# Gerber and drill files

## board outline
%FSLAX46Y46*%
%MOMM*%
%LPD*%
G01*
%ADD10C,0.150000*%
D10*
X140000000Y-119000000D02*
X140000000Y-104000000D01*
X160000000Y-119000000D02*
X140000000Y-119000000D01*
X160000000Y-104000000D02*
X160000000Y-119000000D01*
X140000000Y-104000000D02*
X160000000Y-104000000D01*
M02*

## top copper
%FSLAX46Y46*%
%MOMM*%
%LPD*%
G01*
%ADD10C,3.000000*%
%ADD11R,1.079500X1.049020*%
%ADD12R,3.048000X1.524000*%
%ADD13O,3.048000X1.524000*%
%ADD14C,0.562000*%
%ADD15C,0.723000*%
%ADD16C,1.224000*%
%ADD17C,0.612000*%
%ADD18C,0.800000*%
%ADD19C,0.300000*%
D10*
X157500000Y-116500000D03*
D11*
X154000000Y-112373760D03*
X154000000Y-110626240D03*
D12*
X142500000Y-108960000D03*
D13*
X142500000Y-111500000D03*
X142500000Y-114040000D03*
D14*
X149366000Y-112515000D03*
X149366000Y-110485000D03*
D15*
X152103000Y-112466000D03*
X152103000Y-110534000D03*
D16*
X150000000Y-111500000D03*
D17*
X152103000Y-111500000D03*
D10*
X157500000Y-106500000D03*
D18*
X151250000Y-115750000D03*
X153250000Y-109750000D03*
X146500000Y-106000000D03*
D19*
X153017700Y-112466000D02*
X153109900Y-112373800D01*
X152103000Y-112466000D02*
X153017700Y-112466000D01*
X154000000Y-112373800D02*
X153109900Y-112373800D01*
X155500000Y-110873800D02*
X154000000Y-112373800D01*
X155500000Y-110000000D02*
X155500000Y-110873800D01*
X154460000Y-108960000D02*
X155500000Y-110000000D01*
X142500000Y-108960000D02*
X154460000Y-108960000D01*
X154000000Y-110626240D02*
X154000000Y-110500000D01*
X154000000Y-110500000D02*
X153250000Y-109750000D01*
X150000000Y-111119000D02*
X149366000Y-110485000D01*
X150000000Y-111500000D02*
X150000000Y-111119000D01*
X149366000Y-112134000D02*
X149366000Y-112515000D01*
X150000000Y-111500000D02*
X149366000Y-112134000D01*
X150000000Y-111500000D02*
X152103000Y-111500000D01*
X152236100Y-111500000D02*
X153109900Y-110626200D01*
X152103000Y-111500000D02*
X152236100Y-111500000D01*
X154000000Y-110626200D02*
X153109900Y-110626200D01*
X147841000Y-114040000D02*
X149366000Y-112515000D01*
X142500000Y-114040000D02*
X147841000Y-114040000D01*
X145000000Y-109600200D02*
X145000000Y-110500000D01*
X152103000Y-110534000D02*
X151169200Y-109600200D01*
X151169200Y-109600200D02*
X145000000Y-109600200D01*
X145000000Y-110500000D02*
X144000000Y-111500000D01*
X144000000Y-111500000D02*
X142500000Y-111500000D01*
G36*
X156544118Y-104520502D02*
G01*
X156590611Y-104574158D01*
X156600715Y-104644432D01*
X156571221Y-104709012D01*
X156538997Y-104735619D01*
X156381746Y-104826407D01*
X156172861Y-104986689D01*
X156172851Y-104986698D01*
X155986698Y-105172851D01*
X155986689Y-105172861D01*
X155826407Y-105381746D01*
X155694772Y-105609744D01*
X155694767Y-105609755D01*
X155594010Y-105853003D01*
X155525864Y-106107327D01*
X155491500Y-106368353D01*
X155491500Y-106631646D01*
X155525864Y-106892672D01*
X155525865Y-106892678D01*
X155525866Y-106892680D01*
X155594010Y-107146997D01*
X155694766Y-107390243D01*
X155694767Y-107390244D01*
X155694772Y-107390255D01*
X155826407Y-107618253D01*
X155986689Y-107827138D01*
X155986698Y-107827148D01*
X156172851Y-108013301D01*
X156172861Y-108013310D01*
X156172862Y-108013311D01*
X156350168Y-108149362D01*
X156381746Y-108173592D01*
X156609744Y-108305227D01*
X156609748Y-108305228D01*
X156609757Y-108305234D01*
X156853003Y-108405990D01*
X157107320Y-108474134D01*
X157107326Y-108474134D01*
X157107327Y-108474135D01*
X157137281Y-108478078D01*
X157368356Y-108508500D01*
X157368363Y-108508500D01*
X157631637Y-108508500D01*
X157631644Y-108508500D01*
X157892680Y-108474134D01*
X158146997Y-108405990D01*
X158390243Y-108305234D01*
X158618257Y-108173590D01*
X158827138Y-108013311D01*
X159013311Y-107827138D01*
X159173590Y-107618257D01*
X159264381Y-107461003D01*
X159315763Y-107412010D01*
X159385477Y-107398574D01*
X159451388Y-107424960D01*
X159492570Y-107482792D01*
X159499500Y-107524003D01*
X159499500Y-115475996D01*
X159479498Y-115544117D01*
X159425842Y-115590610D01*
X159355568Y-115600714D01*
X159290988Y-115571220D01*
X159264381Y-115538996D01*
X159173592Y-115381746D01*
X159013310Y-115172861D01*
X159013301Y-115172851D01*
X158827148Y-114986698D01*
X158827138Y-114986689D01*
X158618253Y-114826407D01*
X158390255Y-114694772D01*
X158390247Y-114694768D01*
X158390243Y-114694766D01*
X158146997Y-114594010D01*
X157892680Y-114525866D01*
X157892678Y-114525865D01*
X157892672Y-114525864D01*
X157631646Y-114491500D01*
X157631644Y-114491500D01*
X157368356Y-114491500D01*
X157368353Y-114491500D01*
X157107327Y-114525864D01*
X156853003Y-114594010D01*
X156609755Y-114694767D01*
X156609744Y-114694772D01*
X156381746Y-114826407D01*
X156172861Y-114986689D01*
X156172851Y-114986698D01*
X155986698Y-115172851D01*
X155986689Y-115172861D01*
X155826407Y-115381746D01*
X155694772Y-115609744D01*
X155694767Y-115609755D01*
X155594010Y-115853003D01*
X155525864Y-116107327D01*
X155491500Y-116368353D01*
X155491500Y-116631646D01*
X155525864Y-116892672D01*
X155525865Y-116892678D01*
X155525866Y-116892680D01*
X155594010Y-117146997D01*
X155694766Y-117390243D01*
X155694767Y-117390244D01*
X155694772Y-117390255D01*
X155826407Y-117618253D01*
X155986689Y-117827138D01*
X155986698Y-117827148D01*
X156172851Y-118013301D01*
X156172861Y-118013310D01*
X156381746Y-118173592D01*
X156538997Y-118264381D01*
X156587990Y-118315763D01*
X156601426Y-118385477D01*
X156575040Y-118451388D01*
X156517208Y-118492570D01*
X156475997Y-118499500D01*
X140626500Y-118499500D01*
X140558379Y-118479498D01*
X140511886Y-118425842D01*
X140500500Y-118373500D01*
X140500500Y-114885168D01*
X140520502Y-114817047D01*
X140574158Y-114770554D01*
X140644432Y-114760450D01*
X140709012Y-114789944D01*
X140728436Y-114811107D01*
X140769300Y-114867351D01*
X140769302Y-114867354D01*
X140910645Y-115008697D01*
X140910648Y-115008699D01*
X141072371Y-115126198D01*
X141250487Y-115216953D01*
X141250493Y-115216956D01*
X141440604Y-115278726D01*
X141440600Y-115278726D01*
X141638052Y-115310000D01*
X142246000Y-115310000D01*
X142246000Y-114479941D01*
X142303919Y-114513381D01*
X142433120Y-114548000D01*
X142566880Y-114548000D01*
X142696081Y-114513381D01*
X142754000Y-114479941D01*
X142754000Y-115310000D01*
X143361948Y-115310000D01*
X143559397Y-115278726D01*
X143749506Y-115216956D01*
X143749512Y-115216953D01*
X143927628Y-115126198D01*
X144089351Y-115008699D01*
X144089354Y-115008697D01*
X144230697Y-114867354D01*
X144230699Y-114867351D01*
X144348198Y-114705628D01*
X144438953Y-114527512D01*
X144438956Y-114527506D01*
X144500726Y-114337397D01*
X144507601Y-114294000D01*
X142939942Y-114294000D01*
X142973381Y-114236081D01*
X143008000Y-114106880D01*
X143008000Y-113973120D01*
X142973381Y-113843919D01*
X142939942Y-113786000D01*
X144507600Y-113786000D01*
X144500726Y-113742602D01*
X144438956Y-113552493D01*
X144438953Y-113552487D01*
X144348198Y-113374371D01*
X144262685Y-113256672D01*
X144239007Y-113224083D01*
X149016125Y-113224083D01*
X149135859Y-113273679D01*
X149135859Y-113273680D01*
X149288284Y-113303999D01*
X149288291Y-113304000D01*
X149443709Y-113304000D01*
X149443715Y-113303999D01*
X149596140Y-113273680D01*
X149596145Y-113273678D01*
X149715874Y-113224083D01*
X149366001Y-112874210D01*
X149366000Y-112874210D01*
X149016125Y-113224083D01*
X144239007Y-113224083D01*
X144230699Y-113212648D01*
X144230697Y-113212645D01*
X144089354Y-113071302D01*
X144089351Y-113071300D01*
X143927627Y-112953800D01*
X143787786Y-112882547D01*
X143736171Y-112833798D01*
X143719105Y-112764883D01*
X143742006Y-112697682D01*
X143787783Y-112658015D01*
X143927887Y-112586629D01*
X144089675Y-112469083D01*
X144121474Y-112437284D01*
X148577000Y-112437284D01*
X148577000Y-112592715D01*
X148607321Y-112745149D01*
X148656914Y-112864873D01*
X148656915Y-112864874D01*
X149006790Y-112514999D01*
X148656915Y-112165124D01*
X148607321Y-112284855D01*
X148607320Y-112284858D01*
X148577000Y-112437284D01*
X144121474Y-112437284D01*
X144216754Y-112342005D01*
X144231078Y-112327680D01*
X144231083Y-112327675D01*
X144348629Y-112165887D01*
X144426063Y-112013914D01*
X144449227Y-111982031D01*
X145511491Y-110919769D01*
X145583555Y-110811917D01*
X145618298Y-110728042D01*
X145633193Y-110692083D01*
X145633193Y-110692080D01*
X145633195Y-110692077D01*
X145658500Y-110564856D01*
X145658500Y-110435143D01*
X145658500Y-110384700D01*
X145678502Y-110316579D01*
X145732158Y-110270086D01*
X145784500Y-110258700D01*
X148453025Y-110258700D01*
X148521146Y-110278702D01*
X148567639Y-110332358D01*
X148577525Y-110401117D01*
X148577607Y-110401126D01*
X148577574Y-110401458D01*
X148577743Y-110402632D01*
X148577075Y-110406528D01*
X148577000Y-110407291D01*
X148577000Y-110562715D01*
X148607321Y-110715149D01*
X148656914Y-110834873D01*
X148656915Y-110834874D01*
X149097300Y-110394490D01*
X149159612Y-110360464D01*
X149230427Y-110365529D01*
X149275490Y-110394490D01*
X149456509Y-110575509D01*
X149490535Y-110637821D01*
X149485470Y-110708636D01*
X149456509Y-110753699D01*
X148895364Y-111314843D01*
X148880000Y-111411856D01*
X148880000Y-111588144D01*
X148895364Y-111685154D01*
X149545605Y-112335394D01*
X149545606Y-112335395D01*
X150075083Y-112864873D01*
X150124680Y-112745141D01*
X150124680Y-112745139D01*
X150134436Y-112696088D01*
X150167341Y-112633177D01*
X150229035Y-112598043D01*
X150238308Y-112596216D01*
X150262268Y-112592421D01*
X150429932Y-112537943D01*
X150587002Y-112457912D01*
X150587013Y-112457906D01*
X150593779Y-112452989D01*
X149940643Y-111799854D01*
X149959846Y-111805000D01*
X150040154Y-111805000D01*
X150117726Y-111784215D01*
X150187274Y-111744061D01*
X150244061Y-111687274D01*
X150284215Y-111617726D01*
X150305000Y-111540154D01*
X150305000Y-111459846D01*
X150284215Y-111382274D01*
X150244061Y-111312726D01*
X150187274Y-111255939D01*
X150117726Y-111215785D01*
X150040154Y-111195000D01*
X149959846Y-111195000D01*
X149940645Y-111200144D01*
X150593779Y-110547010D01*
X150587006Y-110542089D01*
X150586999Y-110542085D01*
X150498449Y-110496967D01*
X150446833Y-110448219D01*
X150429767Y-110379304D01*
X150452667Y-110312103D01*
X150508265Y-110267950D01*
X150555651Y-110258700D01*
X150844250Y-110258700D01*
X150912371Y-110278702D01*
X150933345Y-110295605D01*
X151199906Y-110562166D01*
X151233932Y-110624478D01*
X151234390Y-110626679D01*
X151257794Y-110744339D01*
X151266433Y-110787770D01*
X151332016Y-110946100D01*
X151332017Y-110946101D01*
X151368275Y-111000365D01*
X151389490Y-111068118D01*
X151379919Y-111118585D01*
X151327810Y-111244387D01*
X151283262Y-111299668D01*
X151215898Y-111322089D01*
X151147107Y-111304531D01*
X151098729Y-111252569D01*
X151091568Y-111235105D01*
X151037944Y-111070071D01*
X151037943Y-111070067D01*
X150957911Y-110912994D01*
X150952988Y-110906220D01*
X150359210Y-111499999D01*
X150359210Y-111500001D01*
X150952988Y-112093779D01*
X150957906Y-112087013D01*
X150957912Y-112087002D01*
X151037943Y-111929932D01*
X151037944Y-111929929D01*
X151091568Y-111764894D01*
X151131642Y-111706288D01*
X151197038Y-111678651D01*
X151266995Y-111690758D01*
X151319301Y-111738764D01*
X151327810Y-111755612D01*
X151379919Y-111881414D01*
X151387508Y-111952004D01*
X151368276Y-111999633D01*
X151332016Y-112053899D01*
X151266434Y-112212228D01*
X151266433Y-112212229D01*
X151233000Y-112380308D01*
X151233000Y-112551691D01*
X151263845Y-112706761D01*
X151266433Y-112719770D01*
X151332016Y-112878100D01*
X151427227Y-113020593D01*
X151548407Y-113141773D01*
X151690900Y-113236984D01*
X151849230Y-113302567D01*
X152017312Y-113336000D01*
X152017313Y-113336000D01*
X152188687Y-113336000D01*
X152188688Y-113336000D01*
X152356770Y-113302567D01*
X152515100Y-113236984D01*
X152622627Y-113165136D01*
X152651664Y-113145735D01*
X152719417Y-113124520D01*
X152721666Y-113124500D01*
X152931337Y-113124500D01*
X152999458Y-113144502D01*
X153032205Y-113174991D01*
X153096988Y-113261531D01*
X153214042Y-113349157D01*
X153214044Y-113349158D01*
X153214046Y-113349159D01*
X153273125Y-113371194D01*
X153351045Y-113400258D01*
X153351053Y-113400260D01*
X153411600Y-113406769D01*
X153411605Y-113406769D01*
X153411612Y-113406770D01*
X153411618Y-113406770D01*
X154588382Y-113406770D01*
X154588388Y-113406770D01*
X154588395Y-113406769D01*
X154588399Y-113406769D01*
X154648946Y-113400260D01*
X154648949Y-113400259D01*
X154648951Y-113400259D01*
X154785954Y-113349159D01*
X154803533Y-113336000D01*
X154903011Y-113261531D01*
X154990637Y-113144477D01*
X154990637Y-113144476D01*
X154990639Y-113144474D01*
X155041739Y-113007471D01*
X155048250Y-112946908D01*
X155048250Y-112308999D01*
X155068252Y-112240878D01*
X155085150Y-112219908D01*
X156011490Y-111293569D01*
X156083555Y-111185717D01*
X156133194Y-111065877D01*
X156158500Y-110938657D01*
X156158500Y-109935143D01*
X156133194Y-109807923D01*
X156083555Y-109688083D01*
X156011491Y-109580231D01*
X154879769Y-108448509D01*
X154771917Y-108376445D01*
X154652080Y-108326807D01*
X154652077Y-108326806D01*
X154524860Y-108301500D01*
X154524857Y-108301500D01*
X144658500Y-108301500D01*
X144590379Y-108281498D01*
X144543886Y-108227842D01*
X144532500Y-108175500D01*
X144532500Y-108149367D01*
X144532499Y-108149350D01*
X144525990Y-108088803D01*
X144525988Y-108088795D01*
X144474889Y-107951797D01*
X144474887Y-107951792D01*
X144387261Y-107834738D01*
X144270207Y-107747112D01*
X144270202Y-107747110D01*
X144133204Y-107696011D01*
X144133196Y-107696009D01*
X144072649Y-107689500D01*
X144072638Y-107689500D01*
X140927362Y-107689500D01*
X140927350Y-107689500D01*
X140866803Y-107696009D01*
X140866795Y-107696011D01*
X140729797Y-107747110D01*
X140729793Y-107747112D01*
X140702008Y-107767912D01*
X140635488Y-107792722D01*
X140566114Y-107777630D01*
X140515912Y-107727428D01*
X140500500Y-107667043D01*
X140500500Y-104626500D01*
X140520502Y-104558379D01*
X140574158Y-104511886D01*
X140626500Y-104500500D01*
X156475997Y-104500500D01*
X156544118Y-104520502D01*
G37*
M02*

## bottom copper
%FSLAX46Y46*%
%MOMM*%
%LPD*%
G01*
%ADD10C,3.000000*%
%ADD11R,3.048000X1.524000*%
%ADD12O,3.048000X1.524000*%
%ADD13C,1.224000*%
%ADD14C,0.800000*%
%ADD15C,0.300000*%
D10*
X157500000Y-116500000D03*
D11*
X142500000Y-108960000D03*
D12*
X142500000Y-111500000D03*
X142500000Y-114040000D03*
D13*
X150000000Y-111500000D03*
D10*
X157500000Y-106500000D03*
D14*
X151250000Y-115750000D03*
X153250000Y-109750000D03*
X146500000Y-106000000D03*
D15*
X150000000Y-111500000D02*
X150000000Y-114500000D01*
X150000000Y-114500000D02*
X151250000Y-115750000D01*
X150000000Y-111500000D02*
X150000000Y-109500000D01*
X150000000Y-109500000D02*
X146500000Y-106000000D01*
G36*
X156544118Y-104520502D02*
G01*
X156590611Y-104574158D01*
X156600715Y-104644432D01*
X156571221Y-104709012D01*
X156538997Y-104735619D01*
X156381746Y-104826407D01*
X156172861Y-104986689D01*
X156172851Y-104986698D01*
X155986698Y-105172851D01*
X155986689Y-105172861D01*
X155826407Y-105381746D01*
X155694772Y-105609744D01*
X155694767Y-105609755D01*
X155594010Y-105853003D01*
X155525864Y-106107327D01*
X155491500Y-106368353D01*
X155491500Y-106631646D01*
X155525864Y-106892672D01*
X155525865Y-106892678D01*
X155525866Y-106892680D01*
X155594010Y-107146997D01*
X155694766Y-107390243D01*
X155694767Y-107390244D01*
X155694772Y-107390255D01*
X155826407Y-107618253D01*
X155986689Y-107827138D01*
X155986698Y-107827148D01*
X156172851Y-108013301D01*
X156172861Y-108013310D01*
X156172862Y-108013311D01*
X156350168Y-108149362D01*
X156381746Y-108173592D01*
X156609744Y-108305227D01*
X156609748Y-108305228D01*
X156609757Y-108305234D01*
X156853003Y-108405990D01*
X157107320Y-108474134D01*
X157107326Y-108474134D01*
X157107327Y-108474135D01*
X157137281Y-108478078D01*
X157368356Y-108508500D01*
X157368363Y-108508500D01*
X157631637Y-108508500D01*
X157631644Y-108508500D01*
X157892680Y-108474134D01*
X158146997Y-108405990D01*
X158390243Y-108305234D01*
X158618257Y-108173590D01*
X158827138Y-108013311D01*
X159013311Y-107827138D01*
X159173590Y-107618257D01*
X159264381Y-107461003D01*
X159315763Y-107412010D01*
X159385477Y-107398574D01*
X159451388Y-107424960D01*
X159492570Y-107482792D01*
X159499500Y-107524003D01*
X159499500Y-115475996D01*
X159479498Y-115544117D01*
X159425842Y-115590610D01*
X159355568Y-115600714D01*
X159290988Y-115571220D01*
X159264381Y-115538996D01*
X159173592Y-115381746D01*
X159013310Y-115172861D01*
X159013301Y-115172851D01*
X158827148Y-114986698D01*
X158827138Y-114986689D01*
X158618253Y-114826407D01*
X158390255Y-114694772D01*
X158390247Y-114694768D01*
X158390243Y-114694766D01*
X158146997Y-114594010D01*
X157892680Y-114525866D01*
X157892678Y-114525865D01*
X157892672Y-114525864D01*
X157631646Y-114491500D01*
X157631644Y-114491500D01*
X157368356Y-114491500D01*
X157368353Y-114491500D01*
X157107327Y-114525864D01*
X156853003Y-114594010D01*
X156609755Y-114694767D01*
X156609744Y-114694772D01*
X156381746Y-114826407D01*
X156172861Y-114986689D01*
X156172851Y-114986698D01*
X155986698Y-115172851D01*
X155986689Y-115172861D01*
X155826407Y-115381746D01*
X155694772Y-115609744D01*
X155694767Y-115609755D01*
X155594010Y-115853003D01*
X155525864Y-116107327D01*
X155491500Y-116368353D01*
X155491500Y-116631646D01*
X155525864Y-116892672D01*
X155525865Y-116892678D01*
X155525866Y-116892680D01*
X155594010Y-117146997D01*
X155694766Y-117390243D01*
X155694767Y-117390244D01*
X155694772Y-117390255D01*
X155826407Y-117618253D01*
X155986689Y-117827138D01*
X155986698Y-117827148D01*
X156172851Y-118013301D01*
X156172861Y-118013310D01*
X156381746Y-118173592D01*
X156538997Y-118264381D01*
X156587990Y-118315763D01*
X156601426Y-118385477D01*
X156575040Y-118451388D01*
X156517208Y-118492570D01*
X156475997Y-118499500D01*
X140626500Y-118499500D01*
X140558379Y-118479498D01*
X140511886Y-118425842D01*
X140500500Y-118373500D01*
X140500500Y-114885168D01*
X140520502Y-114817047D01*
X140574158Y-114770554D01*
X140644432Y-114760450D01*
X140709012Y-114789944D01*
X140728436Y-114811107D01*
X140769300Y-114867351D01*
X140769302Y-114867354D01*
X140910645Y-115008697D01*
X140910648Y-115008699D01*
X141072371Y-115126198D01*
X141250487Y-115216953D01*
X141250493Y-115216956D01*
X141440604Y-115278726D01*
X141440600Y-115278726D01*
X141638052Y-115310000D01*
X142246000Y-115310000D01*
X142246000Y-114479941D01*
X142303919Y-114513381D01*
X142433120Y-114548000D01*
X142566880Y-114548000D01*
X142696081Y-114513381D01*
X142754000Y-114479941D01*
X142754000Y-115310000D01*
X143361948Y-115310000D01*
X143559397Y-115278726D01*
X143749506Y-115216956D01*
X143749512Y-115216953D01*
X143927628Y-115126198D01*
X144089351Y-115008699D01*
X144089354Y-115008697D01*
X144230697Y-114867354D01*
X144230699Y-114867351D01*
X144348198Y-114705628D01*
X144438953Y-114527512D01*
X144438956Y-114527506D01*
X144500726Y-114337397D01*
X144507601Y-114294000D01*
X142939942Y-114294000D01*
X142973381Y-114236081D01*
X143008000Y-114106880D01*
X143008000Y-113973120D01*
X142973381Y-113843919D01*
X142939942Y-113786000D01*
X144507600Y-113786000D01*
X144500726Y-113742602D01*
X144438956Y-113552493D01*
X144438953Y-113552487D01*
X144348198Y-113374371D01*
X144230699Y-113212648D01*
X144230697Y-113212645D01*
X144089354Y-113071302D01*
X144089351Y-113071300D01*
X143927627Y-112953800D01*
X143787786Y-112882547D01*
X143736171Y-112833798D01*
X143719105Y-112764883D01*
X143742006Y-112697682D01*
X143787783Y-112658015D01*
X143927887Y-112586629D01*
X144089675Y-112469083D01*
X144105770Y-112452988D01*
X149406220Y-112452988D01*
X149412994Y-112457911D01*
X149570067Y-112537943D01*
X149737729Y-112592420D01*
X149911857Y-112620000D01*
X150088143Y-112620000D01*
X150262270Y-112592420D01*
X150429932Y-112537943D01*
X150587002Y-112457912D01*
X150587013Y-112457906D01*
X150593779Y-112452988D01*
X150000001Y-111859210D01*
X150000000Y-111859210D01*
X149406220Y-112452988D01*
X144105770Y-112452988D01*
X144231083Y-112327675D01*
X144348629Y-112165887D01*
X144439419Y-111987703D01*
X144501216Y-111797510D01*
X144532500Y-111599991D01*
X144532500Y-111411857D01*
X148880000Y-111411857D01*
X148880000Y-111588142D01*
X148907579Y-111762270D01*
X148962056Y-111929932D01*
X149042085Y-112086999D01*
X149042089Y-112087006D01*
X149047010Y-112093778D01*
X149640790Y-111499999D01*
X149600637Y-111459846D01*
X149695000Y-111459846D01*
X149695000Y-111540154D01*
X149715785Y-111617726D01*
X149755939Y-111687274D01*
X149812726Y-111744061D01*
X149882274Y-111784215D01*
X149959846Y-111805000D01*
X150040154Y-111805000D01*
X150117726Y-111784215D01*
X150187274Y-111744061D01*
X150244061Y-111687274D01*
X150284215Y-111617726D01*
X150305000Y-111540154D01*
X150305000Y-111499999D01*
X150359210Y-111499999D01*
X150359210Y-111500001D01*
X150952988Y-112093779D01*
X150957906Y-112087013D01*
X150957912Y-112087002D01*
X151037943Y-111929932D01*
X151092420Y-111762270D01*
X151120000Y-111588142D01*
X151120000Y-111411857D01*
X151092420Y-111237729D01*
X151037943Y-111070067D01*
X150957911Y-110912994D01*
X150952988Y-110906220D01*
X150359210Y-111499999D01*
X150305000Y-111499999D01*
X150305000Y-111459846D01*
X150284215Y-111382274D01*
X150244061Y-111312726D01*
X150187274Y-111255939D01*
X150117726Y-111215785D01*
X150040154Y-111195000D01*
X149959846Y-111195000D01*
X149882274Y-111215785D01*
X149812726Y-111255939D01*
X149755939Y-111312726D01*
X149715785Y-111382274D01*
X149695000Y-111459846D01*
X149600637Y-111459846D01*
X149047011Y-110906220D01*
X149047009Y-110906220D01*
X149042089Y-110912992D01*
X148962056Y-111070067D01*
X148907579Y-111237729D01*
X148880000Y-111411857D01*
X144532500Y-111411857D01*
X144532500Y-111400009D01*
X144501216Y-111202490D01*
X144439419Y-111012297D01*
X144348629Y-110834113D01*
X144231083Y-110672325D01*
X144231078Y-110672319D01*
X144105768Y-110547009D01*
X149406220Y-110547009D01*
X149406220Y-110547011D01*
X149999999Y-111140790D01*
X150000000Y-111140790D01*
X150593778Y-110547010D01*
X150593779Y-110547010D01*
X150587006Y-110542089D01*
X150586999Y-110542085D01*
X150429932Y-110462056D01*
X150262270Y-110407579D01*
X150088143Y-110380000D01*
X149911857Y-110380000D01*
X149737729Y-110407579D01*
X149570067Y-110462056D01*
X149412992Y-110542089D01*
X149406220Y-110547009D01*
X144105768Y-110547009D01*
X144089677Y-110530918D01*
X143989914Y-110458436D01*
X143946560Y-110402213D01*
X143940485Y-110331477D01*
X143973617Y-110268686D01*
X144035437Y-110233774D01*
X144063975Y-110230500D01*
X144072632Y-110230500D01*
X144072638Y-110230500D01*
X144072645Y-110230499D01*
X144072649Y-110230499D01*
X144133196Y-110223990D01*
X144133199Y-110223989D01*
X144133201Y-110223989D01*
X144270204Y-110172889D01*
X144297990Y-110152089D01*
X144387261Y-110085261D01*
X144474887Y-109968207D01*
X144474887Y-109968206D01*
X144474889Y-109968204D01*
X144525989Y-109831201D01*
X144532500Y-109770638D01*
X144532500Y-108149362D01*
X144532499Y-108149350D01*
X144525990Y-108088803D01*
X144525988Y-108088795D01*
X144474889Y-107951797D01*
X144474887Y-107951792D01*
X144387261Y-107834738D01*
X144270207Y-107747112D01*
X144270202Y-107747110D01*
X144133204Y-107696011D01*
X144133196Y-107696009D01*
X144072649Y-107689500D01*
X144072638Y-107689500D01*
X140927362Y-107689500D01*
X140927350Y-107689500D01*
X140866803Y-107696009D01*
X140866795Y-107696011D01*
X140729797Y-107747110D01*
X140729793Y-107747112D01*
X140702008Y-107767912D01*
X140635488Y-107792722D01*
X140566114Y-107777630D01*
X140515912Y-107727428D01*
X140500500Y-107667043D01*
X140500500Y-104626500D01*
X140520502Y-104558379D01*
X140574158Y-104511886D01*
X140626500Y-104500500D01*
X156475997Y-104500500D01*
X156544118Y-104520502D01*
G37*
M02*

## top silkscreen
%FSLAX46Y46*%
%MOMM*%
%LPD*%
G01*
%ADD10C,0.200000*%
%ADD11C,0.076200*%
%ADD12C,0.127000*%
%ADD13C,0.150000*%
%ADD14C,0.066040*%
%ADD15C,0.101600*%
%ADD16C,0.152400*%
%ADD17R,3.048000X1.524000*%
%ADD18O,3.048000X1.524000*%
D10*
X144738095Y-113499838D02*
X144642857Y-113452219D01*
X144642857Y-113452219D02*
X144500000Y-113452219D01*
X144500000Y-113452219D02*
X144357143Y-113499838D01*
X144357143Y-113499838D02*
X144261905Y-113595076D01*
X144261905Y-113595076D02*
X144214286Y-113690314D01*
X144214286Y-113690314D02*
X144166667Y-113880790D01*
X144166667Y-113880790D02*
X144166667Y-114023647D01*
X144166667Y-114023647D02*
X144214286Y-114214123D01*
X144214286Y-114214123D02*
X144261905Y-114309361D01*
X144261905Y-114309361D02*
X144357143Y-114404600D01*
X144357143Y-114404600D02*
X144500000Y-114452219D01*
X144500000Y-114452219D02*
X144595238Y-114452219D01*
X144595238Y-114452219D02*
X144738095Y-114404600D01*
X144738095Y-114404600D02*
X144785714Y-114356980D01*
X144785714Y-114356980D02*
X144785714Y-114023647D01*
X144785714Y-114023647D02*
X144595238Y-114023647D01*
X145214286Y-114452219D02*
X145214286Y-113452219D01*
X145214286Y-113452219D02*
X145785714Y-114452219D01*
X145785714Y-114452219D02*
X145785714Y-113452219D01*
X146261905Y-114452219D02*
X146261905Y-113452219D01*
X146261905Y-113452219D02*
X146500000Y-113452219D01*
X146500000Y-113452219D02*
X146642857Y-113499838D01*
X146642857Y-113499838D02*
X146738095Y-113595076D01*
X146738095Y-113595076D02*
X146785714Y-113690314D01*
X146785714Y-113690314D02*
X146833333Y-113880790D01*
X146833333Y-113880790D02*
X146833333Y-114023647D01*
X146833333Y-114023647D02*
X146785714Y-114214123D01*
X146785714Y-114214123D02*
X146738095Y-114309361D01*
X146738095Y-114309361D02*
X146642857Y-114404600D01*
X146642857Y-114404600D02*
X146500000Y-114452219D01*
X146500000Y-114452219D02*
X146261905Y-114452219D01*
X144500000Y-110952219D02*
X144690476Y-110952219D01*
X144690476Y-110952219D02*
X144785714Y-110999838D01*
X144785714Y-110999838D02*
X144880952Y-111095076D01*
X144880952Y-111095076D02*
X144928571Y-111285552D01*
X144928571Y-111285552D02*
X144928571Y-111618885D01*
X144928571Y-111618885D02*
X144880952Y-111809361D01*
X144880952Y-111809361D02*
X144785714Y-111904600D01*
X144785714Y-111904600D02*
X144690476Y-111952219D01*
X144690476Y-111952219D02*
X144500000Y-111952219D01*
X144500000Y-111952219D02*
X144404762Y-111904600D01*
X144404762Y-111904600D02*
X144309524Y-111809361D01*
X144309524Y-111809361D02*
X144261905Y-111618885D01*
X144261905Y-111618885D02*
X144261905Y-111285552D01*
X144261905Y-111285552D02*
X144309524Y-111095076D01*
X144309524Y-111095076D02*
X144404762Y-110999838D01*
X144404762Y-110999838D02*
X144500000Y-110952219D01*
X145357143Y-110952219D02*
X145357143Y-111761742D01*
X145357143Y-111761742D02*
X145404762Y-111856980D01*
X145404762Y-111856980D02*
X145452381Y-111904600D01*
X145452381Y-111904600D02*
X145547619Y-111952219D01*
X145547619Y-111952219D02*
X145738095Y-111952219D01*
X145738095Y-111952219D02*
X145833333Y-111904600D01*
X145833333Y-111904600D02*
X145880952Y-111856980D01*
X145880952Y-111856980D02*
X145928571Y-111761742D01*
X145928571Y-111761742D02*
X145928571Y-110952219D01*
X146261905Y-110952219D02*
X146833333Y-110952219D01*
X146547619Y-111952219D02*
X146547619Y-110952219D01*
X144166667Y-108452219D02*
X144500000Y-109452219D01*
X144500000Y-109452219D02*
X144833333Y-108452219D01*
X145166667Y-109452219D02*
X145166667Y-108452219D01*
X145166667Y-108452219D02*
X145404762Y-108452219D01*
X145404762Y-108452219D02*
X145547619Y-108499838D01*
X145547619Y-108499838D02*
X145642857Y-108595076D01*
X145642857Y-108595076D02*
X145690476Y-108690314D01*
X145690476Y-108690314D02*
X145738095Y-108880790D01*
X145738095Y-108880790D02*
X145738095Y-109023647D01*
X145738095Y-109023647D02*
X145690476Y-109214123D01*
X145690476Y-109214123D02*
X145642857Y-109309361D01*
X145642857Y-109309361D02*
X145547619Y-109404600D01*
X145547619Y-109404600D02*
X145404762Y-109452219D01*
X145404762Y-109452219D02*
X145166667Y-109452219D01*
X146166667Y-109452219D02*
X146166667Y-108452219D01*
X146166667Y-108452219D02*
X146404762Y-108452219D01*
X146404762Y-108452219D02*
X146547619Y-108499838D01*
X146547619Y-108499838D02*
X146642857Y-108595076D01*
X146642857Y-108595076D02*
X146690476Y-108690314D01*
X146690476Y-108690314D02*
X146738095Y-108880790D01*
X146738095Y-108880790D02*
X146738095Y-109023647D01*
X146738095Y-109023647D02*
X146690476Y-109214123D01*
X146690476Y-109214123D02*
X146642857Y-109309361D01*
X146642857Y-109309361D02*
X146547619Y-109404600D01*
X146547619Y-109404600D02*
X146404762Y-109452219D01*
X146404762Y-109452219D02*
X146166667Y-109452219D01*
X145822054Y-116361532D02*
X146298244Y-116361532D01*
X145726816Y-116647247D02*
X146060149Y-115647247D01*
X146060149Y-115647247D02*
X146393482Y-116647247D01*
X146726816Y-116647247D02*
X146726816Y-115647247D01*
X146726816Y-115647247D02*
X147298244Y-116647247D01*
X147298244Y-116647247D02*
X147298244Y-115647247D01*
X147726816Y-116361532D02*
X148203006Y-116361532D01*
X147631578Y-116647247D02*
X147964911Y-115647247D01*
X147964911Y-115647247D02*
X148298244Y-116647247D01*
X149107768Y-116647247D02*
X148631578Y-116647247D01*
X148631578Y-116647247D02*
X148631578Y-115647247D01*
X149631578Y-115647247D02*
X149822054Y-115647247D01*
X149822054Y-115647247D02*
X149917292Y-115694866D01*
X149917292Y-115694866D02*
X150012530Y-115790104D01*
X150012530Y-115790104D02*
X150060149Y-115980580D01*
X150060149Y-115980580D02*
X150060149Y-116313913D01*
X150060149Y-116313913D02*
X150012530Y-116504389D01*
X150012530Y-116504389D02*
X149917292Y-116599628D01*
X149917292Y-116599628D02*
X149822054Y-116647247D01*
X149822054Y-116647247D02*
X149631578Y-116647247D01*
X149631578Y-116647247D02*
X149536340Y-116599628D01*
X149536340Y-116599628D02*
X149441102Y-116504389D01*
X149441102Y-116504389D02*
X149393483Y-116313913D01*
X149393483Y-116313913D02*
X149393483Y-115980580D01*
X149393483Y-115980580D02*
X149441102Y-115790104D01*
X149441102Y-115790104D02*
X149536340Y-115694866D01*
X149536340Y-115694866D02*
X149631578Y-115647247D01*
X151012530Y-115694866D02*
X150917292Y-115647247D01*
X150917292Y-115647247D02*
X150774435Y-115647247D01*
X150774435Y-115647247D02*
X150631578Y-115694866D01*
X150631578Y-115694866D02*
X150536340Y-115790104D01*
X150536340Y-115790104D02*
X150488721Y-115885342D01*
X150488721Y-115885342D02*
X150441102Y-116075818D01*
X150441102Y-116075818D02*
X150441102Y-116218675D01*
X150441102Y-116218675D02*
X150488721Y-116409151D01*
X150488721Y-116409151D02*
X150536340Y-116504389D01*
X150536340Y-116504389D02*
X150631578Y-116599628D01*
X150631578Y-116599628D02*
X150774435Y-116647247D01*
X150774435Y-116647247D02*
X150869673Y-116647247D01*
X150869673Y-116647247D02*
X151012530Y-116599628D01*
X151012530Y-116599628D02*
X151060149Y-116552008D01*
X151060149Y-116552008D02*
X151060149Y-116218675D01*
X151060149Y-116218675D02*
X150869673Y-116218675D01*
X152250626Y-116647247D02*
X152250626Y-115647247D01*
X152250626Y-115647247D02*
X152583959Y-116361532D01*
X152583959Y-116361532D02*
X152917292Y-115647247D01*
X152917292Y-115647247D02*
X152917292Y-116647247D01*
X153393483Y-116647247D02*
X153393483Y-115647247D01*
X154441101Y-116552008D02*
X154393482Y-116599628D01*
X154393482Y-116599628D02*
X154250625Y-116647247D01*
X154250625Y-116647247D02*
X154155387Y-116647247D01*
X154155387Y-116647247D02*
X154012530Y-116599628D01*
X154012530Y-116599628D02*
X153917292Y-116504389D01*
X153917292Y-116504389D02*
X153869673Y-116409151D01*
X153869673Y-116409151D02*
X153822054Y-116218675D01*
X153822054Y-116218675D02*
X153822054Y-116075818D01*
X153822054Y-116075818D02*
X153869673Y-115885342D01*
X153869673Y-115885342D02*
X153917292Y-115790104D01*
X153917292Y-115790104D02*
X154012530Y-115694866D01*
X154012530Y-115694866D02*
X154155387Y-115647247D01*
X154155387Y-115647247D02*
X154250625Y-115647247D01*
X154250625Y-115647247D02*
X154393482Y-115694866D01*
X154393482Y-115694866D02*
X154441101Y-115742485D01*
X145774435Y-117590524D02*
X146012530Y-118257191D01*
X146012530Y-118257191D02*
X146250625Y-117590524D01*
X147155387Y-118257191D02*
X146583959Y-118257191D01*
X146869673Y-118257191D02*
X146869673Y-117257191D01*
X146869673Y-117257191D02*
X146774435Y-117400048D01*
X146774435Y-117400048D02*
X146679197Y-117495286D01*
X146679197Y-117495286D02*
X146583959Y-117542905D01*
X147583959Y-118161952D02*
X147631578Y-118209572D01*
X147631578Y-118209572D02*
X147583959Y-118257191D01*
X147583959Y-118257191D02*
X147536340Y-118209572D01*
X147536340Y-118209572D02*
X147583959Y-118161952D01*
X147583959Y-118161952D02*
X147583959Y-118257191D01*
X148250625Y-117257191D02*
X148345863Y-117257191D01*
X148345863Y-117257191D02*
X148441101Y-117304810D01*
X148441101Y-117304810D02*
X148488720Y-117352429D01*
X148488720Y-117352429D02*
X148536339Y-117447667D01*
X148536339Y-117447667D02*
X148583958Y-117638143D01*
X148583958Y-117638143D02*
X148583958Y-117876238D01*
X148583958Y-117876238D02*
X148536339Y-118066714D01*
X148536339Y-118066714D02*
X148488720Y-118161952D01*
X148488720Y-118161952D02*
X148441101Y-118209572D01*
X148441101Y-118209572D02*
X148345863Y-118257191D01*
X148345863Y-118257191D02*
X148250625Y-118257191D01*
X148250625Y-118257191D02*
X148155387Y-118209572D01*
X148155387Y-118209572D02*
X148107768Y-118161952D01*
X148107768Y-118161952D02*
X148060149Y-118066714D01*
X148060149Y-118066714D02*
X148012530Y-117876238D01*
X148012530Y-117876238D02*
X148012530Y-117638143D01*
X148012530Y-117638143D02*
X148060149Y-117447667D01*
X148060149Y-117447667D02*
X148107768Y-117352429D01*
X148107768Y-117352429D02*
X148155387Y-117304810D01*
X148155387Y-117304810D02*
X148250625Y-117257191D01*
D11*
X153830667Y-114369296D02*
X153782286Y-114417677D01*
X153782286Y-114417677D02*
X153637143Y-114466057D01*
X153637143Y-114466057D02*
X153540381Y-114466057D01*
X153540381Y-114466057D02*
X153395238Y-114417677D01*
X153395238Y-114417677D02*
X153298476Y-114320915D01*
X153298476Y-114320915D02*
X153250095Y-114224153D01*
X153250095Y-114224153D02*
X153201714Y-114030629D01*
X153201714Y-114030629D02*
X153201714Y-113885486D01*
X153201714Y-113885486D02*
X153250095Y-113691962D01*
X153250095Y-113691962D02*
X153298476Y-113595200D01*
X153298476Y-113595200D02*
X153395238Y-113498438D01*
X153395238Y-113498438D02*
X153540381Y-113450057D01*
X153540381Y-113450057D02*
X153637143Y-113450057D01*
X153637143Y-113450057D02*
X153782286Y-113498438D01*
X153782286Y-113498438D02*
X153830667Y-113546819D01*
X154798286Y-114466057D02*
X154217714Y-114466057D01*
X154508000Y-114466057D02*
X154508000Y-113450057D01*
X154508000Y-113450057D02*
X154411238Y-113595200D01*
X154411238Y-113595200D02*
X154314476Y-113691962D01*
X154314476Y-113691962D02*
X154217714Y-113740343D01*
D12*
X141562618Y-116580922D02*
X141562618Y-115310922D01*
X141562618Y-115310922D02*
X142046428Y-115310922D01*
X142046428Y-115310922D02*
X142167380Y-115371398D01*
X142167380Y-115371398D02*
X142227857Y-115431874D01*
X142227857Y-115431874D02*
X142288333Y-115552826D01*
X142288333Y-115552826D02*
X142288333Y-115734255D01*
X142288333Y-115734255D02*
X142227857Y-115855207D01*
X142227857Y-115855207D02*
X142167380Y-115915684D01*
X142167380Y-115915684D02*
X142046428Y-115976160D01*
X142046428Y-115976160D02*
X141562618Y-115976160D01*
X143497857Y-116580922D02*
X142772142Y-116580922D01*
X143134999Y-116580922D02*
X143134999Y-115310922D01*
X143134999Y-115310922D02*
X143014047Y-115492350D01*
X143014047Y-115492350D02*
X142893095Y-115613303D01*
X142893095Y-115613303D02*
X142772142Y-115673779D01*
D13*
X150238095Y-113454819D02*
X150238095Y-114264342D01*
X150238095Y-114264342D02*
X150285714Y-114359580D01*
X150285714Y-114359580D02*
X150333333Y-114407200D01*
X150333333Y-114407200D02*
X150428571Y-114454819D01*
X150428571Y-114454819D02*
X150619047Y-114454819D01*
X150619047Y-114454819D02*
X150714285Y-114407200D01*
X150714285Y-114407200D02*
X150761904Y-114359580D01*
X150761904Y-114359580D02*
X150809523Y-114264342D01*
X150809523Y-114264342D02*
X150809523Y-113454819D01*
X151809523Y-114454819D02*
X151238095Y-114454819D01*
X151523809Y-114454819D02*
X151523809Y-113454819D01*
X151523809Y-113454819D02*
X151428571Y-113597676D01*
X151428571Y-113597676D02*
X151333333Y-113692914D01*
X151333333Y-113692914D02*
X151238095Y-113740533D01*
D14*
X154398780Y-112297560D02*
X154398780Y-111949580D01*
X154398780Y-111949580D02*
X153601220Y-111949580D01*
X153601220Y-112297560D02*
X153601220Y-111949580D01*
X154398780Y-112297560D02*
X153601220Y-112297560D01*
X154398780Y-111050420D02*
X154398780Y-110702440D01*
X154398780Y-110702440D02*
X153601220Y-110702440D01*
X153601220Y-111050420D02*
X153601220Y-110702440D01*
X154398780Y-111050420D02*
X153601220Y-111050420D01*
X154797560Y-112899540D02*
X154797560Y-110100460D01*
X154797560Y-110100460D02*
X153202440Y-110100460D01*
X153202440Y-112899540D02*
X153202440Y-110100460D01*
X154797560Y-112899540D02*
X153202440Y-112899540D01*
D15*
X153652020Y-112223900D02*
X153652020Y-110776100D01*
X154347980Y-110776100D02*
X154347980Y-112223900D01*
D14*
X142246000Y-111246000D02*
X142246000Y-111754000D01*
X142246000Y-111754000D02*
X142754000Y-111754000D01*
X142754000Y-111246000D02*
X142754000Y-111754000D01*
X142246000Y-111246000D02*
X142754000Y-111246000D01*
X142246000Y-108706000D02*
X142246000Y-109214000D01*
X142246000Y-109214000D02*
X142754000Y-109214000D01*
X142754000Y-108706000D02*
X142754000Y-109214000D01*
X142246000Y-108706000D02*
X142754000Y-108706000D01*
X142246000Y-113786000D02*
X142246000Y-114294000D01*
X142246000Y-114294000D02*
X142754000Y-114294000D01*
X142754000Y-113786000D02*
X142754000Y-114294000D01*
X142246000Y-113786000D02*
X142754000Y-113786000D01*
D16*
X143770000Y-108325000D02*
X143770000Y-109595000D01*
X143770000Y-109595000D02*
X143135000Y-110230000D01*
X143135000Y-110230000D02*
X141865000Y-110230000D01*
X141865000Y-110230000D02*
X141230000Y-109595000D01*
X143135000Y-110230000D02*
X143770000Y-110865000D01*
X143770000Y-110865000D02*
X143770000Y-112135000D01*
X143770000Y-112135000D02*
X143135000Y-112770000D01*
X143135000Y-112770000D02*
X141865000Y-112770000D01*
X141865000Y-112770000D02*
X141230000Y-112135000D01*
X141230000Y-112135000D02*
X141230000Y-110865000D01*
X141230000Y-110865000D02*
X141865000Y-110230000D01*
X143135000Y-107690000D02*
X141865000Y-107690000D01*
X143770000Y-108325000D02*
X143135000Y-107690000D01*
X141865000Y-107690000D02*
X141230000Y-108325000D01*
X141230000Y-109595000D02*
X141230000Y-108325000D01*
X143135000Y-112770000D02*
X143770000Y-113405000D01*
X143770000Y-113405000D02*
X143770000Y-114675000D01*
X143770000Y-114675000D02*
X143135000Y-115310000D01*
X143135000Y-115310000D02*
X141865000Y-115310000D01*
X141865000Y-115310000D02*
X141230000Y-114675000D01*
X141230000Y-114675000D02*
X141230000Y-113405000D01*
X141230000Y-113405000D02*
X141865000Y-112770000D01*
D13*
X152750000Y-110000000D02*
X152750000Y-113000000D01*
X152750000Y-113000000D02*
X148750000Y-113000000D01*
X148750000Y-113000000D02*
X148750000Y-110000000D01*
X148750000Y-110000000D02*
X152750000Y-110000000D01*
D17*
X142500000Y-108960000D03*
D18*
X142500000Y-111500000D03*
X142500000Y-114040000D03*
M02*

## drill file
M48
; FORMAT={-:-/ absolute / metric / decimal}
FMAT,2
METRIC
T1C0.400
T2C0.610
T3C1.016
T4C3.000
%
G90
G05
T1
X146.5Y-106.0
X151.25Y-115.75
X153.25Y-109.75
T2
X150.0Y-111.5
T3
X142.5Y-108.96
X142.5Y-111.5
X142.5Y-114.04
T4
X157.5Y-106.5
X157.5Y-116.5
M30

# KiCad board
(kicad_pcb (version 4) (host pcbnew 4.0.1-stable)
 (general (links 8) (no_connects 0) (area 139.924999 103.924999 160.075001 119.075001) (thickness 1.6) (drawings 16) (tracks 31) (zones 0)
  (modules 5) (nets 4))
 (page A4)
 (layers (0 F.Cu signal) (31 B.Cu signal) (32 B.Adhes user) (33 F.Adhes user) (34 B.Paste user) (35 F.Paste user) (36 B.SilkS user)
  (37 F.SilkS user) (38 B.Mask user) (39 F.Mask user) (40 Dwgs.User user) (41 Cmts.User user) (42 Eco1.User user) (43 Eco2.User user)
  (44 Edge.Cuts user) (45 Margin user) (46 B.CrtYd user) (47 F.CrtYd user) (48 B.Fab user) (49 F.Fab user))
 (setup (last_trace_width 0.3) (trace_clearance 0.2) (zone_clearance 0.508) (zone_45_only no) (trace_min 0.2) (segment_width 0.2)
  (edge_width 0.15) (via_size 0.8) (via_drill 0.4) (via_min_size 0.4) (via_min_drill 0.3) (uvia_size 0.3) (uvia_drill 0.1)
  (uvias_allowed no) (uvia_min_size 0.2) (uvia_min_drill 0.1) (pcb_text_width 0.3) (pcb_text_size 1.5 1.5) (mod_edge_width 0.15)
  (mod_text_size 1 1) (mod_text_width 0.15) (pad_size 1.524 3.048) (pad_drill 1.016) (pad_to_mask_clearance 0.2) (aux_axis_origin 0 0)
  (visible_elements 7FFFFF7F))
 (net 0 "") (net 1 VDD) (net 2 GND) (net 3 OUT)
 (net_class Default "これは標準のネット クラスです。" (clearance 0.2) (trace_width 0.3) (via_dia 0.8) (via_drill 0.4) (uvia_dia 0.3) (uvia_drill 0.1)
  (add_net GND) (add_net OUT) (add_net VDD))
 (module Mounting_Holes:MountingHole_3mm (layer F.Cu) (at 157.5 116.5)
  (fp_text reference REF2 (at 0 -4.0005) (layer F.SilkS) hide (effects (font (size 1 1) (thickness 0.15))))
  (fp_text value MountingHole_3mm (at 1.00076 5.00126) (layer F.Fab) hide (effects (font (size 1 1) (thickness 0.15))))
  (pad 1 thru_hole circle (at 0 0) (size 3 3) (drill 3) (layers)))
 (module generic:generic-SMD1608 (layer F.Cu) (at 154 111.5 90)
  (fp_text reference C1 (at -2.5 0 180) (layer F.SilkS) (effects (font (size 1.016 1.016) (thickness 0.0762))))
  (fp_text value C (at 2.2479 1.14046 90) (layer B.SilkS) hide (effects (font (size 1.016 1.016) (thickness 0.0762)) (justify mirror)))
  (fp_line (start -0.79756 0.39878) (end -0.44958 0.39878) (layer F.SilkS) (width 0.06604))
  (fp_line (start -0.44958 0.39878) (end -0.44958 -0.39878) (layer F.SilkS) (width 0.06604))
  (fp_line (start -0.79756 -0.39878) (end -0.44958 -0.39878) (layer F.SilkS) (width 0.06604))
  (fp_line (start -0.79756 0.39878) (end -0.79756 -0.39878) (layer F.SilkS) (width 0.06604))
  (fp_line (start 0.44958 0.39878) (end 0.79756 0.39878) (layer F.SilkS) (width 0.06604))
  (fp_line (start 0.79756 0.39878) (end 0.79756 -0.39878) (layer F.SilkS) (width 0.06604))
  (fp_line (start 0.44958 -0.39878) (end 0.79756 -0.39878) (layer F.SilkS) (width 0.06604))
  (fp_line (start 0.44958 0.39878) (end 0.44958 -0.39878) (layer F.SilkS) (width 0.06604))
  (fp_line (start -1.39954 0.79756) (end 1.39954 0.79756) (layer F.SilkS) (width 0.06604))
  (fp_line (start 1.39954 0.79756) (end 1.39954 -0.79756) (layer F.SilkS) (width 0.06604))
  (fp_line (start -1.39954 -0.79756) (end 1.39954 -0.79756) (layer F.SilkS) (width 0.06604))
  (fp_line (start -1.39954 0.79756) (end -1.39954 -0.79756) (layer F.SilkS) (width 0.06604))
  (fp_line (start -0.7239 -0.34798) (end 0.7239 -0.34798) (layer F.SilkS) (width 0.1016))
  (fp_line (start 0.7239 0.34798) (end -0.7239 0.34798) (layer F.SilkS) (width 0.1016))
  (pad 1 smd rect (at -0.87376 0 90) (size 1.04902 1.0795) (layers F.Cu F.Paste F.Mask) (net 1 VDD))
  (pad 2 smd rect (at 0.87376 0 90) (size 1.04902 1.0795) (layers F.Cu F.Paste F.Mask) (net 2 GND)))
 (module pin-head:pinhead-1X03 (layer F.Cu) (at 142.5 111.5 270)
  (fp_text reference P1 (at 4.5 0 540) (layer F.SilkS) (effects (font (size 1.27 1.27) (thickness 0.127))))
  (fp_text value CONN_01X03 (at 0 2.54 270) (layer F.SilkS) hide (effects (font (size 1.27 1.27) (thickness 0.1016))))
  (fp_line (start -0.254 0.254) (end 0.254 0.254) (layer F.SilkS) (width 0.06604))
  (fp_line (start 0.254 0.254) (end 0.254 -0.254) (layer F.SilkS) (width 0.06604))
  (fp_line (start -0.254 -0.254) (end 0.254 -0.254) (layer F.SilkS) (width 0.06604))
  (fp_line (start -0.254 0.254) (end -0.254 -0.254) (layer F.SilkS) (width 0.06604))
  (fp_line (start -2.794 0.254) (end -2.286 0.254) (layer F.SilkS) (width 0.06604))
  (fp_line (start -2.286 0.254) (end -2.286 -0.254) (layer F.SilkS) (width 0.06604))
  (fp_line (start -2.794 -0.254) (end -2.286 -0.254) (layer F.SilkS) (width 0.06604))
  (fp_line (start -2.794 0.254) (end -2.794 -0.254) (layer F.SilkS) (width 0.06604))
  (fp_line (start 2.286 0.254) (end 2.794 0.254) (layer F.SilkS) (width 0.06604))
  (fp_line (start 2.794 0.254) (end 2.794 -0.254) (layer F.SilkS) (width 0.06604))
  (fp_line (start 2.286 -0.254) (end 2.794 -0.254) (layer F.SilkS) (width 0.06604))
  (fp_line (start 2.286 0.254) (end 2.286 -0.254) (layer F.SilkS) (width 0.06604))
  (fp_line (start -3.175 -1.27) (end -1.905 -1.27) (layer F.SilkS) (width 0.1524))
  (fp_line (start -1.905 -1.27) (end -1.27 -0.635) (layer F.SilkS) (width 0.1524))
  (fp_line (start -1.27 -0.635) (end -1.27 0.635) (layer F.SilkS) (width 0.1524))
  (fp_line (start -1.27 0.635) (end -1.905 1.27) (layer F.SilkS) (width 0.1524))
  (fp_line (start -1.27 -0.635) (end -0.635 -1.27) (layer F.SilkS) (width 0.1524))
  (fp_line (start -0.635 -1.27) (end 0.635 -1.27) (layer F.SilkS) (width 0.1524))
  (fp_line (start 0.635 -1.27) (end 1.27 -0.635) (layer F.SilkS) (width 0.1524))
  (fp_line (start 1.27 -0.635) (end 1.27 0.635) (layer F.SilkS) (width 0.1524))
  (fp_line (start 1.27 0.635) (end 0.635 1.27) (layer F.SilkS) (width 0.1524))
  (fp_line (start 0.635 1.27) (end -0.635 1.27) (layer F.SilkS) (width 0.1524))
  (fp_line (start -0.635 1.27) (end -1.27 0.635) (layer F.SilkS) (width 0.1524))
  (fp_line (start -3.81 -0.635) (end -3.81 0.635) (layer F.SilkS) (width 0.1524))
  (fp_line (start -3.175 -1.27) (end -3.81 -0.635) (layer F.SilkS) (width 0.1524))
  (fp_line (start -3.81 0.635) (end -3.175 1.27) (layer F.SilkS) (width 0.1524))
  (fp_line (start -1.905 1.27) (end -3.175 1.27) (layer F.SilkS) (width 0.1524))
  (fp_line (start 1.27 -0.635) (end 1.905 -1.27) (layer F.SilkS) (width 0.1524))
  (fp_line (start 1.905 -1.27) (end 3.175 -1.27) (layer F.SilkS) (width 0.1524))
  (fp_line (start 3.175 -1.27) (end 3.81 -0.635) (layer F.SilkS) (width 0.1524))
  (fp_line (start 3.81 -0.635) (end 3.81 0.635) (layer F.SilkS) (width 0.1524))
  (fp_line (start 3.81 0.635) (end 3.175 1.27) (layer F.SilkS) (width 0.1524))
  (fp_line (start 3.175 1.27) (end 1.905 1.27) (layer F.SilkS) (width 0.1524))
  (fp_line (start 1.905 1.27) (end 1.27 0.635) (layer F.SilkS) (width 0.1524))
  (pad 1 thru_hole rect (at -2.54 0 90) (size 1.524 3.048) (drill 1.016) (layers *.Cu *.Paste *.Mask F.SilkS) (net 1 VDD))
  (pad 2 thru_hole oval (at 0 0 90) (size 1.524 3.048) (drill 1.016) (layers *.Cu *.Paste *.Mask F.SilkS) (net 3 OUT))
  (pad 3 thru_hole oval (at 2.54 0 90) (size 1.524 3.048) (drill 1.016) (layers *.Cu *.Paste *.Mask F.SilkS) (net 2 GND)))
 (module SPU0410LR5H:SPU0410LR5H (layer F.Cu) (at 150 111.5 270)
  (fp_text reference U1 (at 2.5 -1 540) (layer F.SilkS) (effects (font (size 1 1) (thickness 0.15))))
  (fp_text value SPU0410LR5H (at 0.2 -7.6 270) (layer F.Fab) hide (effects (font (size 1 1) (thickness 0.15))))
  (fp_line (start -1.5 -2.75) (end 1.5 -2.75) (layer F.SilkS) (width 0.15))
  (fp_line (start 1.5 -2.75) (end 1.5 1.25) (layer F.SilkS) (width 0.15))
  (fp_line (start 1.5 1.25) (end -1.5 1.25) (layer F.SilkS) (width 0.15))
  (fp_line (start -1.5 1.25) (end -1.5 -2.75) (layer F.SilkS) (width 0.15))
  (pad 3 smd circle (at 1.015 0.634 270) (size 0.562 0.562) (layers F.Cu F.Paste F.Mask) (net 2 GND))
  (pad 2 smd circle (at -1.015 0.634 270) (size 0.562 0.562) (layers F.Cu F.Paste F.Mask) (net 2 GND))
  (pad 4 smd circle (at 0.966 -2.103 270) (size 0.723 0.723) (layers F.Cu F.Paste F.Mask) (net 1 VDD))
  (pad 1 smd circle (at -0.966 -2.103 270) (size 0.723 0.723) (layers F.Cu F.Paste F.Mask) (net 3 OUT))
  (pad 6 thru_hole circle (at 0 0 270) (size 1.224 1.224) (drill 0.61) (layers *.Cu F.Paste F.Mask) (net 2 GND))
  (pad 5 smd circle (at 0 -2.103 270) (size 0.612 0.612) (layers F.Cu F.Paste F.Mask) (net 2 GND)))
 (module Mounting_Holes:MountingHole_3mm (layer F.Cu) (at 157.5 106.5)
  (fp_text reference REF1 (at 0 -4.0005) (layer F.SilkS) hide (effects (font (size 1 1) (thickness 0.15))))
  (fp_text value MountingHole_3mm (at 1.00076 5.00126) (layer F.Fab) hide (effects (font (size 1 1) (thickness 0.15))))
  (pad 1 thru_hole circle (at 0 0) (size 3 3) (drill 3) (layers)))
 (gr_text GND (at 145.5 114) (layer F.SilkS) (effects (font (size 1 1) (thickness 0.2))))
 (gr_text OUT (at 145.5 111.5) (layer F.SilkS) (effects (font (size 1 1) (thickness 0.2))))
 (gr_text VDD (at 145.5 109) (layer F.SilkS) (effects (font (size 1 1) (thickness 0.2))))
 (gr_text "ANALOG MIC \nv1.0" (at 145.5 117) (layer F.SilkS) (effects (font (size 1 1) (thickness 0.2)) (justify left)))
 (gr_line (start 140 119) (end 140 104) (angle 90) (layer Edge.Cuts) (width 0.15))
 (gr_line (start 160 119) (end 140 119) (angle 90) (layer Edge.Cuts) (width 0.15))
 (gr_line (start 160 104) (end 160 119) (angle 90) (layer Edge.Cuts) (width 0.15))
 (gr_line (start 140 104) (end 160 104) (angle 90) (layer Edge.Cuts) (width 0.15))
 (segment (start 153.0177 112.466) (end 153.1099 112.3738) (width 0.3) (layer F.Cu) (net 1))
 (segment (start 152.103 112.466) (end 153.0177 112.466) (width 0.3) (layer F.Cu) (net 1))
 (segment (start 154 112.3738) (end 153.1099 112.3738) (width 0.3) (layer F.Cu) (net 1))
 (segment (start 155.5 110.8738) (end 154 112.3738) (width 0.3) (layer F.Cu) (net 1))
 (segment (start 155.5 110) (end 155.5 110.8738) (width 0.3) (layer F.Cu) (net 1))
 (segment (start 154.46 108.96) (end 155.5 110) (width 0.3) (layer F.Cu) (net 1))
 (segment (start 142.5 108.96) (end 154.46 108.96) (width 0.3) (layer F.Cu) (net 1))
 (segment (start 150 111.5) (end 150 114.5) (width 0.3) (layer B.Cu) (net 2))
 (via (at 151.25 115.75) (size 0.8) (drill 0.4) (layers F.Cu B.Cu) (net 2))
 (segment (start 150 114.5) (end 151.25 115.75) (width 0.3) (layer B.Cu) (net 2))
 (segment (start 154 110.62624) (end 154 110.5) (width 0.3) (layer F.Cu) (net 2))
 (segment (start 154 110.5) (end 153.25 109.75) (width 0.3) (layer F.Cu) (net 2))
 (via (at 153.25 109.75) (size 0.8) (drill 0.4) (layers F.Cu B.Cu) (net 2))
 (segment (start 150 111.5) (end 150 109.5) (width 0.3) (layer B.Cu) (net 2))
 (via (at 146.5 106) (size 0.8) (drill 0.4) (layers F.Cu B.Cu) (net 2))
 (segment (start 150 109.5) (end 146.5 106) (width 0.3) (layer B.Cu) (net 2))
 (segment (start 150 111.119) (end 149.366 110.485) (width 0.3) (layer F.Cu) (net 2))
 (segment (start 150 111.5) (end 150 111.119) (width 0.3) (layer F.Cu) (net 2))
 (segment (start 149.366 112.134) (end 149.366 112.515) (width 0.3) (layer F.Cu) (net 2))
 (segment (start 150 111.5) (end 149.366 112.134) (width 0.3) (layer F.Cu) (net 2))
 (segment (start 150 111.5) (end 152.103 111.5) (width 0.3) (layer F.Cu) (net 2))
 (segment (start 152.2361 111.5) (end 153.1099 110.6262) (width 0.3) (layer F.Cu) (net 2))
 (segment (start 152.103 111.5) (end 152.2361 111.5) (width 0.3) (layer F.Cu) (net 2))
 (segment (start 154 110.6262) (end 153.1099 110.6262) (width 0.3) (layer F.Cu) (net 2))
 (segment (start 147.841 114.04) (end 149.366 112.515) (width 0.3) (layer F.Cu) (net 2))
 (segment (start 142.5 114.04) (end 147.841 114.04) (width 0.3) (layer F.Cu) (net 2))
 (segment (start 145 109.6002) (end 145 110.5) (width 0.3) (layer F.Cu) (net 3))
 (segment (start 152.103 110.534) (end 151.1692 109.6002) (width 0.3) (layer F.Cu) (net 3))
 (segment (start 151.1692 109.6002) (end 145 109.6002) (width 0.3) (layer F.Cu) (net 3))
 (segment (start 145 110.5) (end 144 111.5) (width 0.3) (layer F.Cu) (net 3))
 (segment (start 144 111.5) (end 142.5 111.5) (width 0.3) (layer F.Cu) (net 3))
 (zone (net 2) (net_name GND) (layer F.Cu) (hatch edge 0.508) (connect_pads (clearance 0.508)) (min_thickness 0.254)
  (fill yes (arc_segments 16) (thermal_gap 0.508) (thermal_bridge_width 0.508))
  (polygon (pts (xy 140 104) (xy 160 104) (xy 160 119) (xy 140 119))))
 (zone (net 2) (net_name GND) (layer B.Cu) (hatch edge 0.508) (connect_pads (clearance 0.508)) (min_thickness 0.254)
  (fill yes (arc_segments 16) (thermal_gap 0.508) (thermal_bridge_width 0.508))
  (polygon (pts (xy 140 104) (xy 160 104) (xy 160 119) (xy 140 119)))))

